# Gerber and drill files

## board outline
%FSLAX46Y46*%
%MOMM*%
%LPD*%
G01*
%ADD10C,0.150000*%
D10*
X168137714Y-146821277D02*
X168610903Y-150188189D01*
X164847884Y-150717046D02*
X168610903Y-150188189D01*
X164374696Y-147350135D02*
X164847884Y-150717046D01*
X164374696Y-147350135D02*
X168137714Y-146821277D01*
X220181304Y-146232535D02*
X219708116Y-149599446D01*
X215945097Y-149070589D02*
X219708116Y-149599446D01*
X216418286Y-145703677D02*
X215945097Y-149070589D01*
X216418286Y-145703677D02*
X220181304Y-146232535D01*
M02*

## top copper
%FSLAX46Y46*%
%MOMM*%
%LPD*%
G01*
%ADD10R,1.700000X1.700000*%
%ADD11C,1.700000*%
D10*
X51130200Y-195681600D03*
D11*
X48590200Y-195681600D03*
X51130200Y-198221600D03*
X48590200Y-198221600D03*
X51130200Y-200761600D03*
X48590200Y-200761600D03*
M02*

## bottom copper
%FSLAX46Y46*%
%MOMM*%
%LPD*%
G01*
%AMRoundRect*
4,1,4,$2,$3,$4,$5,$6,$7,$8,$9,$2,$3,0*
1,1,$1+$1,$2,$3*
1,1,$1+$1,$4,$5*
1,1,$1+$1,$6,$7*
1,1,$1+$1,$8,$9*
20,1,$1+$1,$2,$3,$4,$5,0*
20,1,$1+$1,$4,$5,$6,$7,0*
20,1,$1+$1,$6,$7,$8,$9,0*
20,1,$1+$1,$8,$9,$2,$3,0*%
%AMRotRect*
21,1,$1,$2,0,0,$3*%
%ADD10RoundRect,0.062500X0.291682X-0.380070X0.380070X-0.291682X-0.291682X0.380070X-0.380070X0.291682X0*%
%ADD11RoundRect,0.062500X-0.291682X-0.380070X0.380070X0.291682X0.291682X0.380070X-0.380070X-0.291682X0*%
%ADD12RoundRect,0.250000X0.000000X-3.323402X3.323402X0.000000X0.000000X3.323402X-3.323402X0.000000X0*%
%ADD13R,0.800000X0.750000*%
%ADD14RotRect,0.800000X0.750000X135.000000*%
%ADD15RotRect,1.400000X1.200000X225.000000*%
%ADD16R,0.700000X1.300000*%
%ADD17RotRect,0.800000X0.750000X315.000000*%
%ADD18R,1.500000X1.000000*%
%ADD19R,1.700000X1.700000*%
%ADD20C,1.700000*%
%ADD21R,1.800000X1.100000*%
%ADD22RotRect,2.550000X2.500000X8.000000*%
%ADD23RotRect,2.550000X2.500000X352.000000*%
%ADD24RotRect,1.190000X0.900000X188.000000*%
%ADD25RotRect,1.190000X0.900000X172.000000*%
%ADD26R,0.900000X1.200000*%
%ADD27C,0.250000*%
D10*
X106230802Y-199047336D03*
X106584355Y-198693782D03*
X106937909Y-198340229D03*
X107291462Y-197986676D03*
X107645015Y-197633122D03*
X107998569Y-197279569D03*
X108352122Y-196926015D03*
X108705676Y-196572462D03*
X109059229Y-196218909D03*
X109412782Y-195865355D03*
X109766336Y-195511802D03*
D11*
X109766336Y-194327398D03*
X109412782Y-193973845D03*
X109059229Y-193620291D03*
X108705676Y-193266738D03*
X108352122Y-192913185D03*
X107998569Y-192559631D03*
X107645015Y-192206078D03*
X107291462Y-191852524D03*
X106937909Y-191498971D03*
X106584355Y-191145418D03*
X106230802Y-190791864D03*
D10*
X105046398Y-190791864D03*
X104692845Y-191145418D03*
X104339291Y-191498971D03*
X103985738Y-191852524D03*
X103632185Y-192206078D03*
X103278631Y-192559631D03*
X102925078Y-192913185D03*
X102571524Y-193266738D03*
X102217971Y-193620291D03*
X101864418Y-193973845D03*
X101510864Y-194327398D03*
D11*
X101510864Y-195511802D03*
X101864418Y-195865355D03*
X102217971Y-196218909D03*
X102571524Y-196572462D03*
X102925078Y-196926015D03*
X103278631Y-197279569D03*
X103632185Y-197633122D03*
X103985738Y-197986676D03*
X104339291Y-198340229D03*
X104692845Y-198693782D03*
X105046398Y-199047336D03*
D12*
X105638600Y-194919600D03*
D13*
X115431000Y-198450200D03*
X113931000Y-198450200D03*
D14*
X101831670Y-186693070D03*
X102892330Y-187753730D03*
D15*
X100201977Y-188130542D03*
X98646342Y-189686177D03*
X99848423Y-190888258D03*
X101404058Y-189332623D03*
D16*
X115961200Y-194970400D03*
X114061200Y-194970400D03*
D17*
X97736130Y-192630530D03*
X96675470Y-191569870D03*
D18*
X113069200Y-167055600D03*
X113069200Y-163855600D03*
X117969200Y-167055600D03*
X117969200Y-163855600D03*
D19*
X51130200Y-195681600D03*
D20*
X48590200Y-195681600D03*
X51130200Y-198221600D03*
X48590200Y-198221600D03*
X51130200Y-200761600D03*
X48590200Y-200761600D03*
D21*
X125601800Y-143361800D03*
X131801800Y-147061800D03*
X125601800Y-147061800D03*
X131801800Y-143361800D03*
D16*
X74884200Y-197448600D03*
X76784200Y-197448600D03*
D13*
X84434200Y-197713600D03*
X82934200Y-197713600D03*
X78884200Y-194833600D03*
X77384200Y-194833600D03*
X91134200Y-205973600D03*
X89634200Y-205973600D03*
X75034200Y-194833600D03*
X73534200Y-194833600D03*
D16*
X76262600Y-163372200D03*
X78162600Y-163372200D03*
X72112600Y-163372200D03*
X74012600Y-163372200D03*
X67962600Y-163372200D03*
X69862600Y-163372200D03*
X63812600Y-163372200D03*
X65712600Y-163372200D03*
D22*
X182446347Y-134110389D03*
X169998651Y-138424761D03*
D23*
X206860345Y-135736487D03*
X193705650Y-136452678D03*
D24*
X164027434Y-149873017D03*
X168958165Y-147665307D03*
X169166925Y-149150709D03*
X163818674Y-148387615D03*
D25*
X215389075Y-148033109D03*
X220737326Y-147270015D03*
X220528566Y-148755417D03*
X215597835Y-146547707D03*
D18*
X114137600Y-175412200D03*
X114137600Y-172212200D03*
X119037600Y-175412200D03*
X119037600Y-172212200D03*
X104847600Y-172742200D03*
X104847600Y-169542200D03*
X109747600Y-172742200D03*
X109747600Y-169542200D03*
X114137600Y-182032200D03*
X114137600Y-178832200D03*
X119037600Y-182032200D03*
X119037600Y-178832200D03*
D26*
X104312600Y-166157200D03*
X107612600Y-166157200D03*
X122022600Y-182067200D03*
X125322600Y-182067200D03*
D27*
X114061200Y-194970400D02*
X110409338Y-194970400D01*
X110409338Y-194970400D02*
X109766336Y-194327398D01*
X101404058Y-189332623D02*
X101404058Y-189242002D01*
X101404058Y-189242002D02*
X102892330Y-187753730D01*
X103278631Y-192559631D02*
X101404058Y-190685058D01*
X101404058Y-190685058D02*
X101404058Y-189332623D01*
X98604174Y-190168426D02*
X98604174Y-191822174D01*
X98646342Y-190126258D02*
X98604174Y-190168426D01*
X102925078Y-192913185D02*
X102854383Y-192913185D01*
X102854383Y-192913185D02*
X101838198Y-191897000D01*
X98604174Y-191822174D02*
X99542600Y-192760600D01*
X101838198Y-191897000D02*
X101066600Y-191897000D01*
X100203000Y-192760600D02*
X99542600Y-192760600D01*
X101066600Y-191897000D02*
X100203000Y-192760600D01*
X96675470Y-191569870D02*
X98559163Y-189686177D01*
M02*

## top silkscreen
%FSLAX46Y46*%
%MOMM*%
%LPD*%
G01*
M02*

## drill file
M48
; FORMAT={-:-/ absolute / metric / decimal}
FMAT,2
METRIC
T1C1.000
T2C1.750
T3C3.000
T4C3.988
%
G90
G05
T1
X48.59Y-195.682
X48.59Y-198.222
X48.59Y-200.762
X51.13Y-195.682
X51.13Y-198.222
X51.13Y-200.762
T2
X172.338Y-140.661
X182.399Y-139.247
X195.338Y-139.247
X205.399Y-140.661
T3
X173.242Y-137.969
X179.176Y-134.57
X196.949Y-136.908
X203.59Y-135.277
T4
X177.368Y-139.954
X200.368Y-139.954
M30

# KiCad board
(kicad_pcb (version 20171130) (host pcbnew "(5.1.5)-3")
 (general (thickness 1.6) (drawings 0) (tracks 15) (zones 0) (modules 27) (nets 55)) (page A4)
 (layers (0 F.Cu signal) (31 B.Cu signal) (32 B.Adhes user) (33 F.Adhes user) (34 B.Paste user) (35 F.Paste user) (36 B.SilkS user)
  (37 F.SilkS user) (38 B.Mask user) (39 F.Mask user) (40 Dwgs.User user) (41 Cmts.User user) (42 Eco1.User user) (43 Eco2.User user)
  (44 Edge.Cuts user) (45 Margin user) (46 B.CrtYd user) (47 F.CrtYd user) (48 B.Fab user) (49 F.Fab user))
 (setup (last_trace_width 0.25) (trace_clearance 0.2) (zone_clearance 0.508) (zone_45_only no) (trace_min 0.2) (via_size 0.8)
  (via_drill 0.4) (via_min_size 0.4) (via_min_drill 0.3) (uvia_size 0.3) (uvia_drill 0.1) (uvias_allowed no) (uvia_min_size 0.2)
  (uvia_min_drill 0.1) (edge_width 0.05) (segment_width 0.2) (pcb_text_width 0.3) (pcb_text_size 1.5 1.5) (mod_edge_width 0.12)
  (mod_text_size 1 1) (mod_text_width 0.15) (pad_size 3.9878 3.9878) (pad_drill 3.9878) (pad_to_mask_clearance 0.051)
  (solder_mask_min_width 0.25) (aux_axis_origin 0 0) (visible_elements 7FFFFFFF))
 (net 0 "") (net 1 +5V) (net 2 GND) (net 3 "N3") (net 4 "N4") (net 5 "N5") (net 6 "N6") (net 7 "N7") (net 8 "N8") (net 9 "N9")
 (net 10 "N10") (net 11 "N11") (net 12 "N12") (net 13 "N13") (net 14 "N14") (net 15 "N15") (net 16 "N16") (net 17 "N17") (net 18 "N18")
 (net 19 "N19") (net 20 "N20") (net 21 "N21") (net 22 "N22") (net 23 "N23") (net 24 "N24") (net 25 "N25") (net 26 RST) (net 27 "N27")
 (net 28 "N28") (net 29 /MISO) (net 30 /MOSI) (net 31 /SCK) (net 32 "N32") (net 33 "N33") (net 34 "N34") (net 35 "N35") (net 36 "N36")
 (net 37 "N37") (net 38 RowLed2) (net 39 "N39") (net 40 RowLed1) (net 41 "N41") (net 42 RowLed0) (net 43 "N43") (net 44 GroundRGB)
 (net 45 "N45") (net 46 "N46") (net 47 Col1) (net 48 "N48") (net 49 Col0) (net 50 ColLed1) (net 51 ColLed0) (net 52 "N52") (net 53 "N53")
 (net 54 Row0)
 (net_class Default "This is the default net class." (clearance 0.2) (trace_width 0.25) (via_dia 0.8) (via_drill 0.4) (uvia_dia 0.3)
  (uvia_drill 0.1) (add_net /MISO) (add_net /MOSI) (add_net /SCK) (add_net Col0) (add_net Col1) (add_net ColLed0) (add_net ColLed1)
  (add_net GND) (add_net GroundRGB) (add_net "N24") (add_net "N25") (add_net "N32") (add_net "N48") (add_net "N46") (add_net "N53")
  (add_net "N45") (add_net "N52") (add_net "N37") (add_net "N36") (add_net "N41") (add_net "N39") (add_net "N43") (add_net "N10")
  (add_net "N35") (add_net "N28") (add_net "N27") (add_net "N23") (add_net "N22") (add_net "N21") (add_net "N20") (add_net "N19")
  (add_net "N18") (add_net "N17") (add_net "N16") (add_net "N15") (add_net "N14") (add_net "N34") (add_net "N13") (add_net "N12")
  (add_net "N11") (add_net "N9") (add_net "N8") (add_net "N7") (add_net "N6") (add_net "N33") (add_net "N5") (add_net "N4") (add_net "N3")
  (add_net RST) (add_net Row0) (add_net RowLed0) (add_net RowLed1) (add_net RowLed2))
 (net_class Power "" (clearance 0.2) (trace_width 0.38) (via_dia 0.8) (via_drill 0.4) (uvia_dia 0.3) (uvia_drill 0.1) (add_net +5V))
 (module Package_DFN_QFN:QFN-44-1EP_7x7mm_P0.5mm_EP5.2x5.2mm (layer B.Cu) (at 105.6386 194.9196 45)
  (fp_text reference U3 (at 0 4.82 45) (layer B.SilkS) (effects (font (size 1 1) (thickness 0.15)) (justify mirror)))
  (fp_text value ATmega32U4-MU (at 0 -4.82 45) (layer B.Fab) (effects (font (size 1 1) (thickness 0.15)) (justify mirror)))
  (pad 44 smd roundrect (at -2.5 3.3375 45) (size 0.25 1.075) (layers B.Cu B.Paste B.Mask) (roundrect_rratio 0.25) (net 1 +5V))
  (pad 43 smd roundrect (at -2 3.3375 45) (size 0.25 1.075) (layers B.Cu B.Paste B.Mask) (roundrect_rratio 0.25) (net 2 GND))
  (pad 42 smd roundrect (at -1.5 3.3375 45) (size 0.25 1.075) (layers B.Cu B.Paste B.Mask) (roundrect_rratio 0.25) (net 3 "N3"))
  (pad 41 smd roundrect (at -1 3.3375 45) (size 0.25 1.075) (layers B.Cu B.Paste B.Mask) (roundrect_rratio 0.25) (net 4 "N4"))
  (pad 40 smd roundrect (at -0.5 3.3375 45) (size 0.25 1.075) (layers B.Cu B.Paste B.Mask) (roundrect_rratio 0.25) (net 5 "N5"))
  (pad 39 smd roundrect (at 0 3.3375 45) (size 0.25 1.075) (layers B.Cu B.Paste B.Mask) (roundrect_rratio 0.25) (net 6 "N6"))
  (pad 38 smd roundrect (at 0.5 3.3375 45) (size 0.25 1.075) (layers B.Cu B.Paste B.Mask) (roundrect_rratio 0.25) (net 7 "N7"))
  (pad 37 smd roundrect (at 1 3.3375 45) (size 0.25 1.075) (layers B.Cu B.Paste B.Mask) (roundrect_rratio 0.25) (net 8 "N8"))
  (pad 36 smd roundrect (at 1.5 3.3375 45) (size 0.25 1.075) (layers B.Cu B.Paste B.Mask) (roundrect_rratio 0.25) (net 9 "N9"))
  (pad 35 smd roundrect (at 2 3.3375 45) (size 0.25 1.075) (layers B.Cu B.Paste B.Mask) (roundrect_rratio 0.25) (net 2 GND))
  (pad 34 smd roundrect (at 2.5 3.3375 45) (size 0.25 1.075) (layers B.Cu B.Paste B.Mask) (roundrect_rratio 0.25) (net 1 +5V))
  (pad 33 smd roundrect (at 3.3375 2.5 45) (size 1.075 0.25) (layers B.Cu B.Paste B.Mask) (roundrect_rratio 0.25) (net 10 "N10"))
  (pad 32 smd roundrect (at 3.3375 2 45) (size 1.075 0.25) (layers B.Cu B.Paste B.Mask) (roundrect_rratio 0.25) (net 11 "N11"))
  (pad 31 smd roundrect (at 3.3375 1.5 45) (size 1.075 0.25) (layers B.Cu B.Paste B.Mask) (roundrect_rratio 0.25) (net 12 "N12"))
  (pad 30 smd roundrect (at 3.3375 1 45) (size 1.075 0.25) (layers B.Cu B.Paste B.Mask) (roundrect_rratio 0.25) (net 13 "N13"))
  (pad 29 smd roundrect (at 3.3375 0.5 45) (size 1.075 0.25) (layers B.Cu B.Paste B.Mask) (roundrect_rratio 0.25) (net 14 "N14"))
  (pad 28 smd roundrect (at 3.3375 0 45) (size 1.075 0.25) (layers B.Cu B.Paste B.Mask) (roundrect_rratio 0.25) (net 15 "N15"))
  (pad 27 smd roundrect (at 3.3375 -0.5 45) (size 1.075 0.25) (layers B.Cu B.Paste B.Mask) (roundrect_rratio 0.25) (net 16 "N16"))
  (pad 26 smd roundrect (at 3.3375 -1 45) (size 1.075 0.25) (layers B.Cu B.Paste B.Mask) (roundrect_rratio 0.25) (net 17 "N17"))
  (pad 25 smd roundrect (at 3.3375 -1.5 45) (size 1.075 0.25) (layers B.Cu B.Paste B.Mask) (roundrect_rratio 0.25) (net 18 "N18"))
  (pad 24 smd roundrect (at 3.3375 -2 45) (size 1.075 0.25) (layers B.Cu B.Paste B.Mask) (roundrect_rratio 0.25) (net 1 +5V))
  (pad 23 smd roundrect (at 3.3375 -2.5 45) (size 1.075 0.25) (layers B.Cu B.Paste B.Mask) (roundrect_rratio 0.25) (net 2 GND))
  (pad 22 smd roundrect (at 2.5 -3.3375 45) (size 0.25 1.075) (layers B.Cu B.Paste B.Mask) (roundrect_rratio 0.25) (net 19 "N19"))
  (pad 21 smd roundrect (at 2 -3.3375 45) (size 0.25 1.075) (layers B.Cu B.Paste B.Mask) (roundrect_rratio 0.25) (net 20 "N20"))
  (pad 20 smd roundrect (at 1.5 -3.3375 45) (size 0.25 1.075) (layers B.Cu B.Paste B.Mask) (roundrect_rratio 0.25) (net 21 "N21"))
  (pad 19 smd roundrect (at 1 -3.3375 45) (size 0.25 1.075) (layers B.Cu B.Paste B.Mask) (roundrect_rratio 0.25) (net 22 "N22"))
  (pad 18 smd roundrect (at 0.5 -3.3375 45) (size 0.25 1.075) (layers B.Cu B.Paste B.Mask) (roundrect_rratio 0.25) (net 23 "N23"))
  (pad 17 smd roundrect (at 0 -3.3375 45) (size 0.25 1.075) (layers B.Cu B.Paste B.Mask) (roundrect_rratio 0.25) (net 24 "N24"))
  (pad 16 smd roundrect (at -0.5 -3.3375 45) (size 0.25 1.075) (layers B.Cu B.Paste B.Mask) (roundrect_rratio 0.25) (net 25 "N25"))
  (pad 15 smd roundrect (at -1 -3.3375 45) (size 0.25 1.075) (layers B.Cu B.Paste B.Mask) (roundrect_rratio 0.25) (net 2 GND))
  (pad 14 smd roundrect (at -1.5 -3.3375 45) (size 0.25 1.075) (layers B.Cu B.Paste B.Mask) (roundrect_rratio 0.25) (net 1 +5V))
  (pad 13 smd roundrect (at -2 -3.3375 45) (size 0.25 1.075) (layers B.Cu B.Paste B.Mask) (roundrect_rratio 0.25) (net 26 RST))
  (pad 12 smd roundrect (at -2.5 -3.3375 45) (size 0.25 1.075) (layers B.Cu B.Paste B.Mask) (roundrect_rratio 0.25) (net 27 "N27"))
  (pad 11 smd roundrect (at -3.3375 -2.5 45) (size 1.075 0.25) (layers B.Cu B.Paste B.Mask) (roundrect_rratio 0.25) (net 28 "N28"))
  (pad 10 smd roundrect (at -3.3375 -2 45) (size 1.075 0.25) (layers B.Cu B.Paste B.Mask) (roundrect_rratio 0.25) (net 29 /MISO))
  (pad 9 smd roundrect (at -3.3375 -1.5 45) (size 1.075 0.25) (layers B.Cu B.Paste B.Mask) (roundrect_rratio 0.25) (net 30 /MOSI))
  (pad 8 smd roundrect (at -3.3375 -1 45) (size 1.075 0.25) (layers B.Cu B.Paste B.Mask) (roundrect_rratio 0.25) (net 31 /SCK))
  (pad 7 smd roundrect (at -3.3375 -0.5 45) (size 1.075 0.25) (layers B.Cu B.Paste B.Mask) (roundrect_rratio 0.25) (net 1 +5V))
  (pad 6 smd roundrect (at -3.3375 0 45) (size 1.075 0.25) (layers B.Cu B.Paste B.Mask) (roundrect_rratio 0.25) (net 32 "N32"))
  (pad 5 smd roundrect (at -3.3375 0.5 45) (size 1.075 0.25) (layers B.Cu B.Paste B.Mask) (roundrect_rratio 0.25) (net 2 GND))
  (pad 4 smd roundrect (at -3.3375 1 45) (size 1.075 0.25) (layers B.Cu B.Paste B.Mask) (roundrect_rratio 0.25) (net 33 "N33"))
  (pad 3 smd roundrect (at -3.3375 1.5 45) (size 1.075 0.25) (layers B.Cu B.Paste B.Mask) (roundrect_rratio 0.25) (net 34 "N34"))
  (pad 2 smd roundrect (at -3.3375 2 45) (size 1.075 0.25) (layers B.Cu B.Paste B.Mask) (roundrect_rratio 0.25) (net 1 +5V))
  (pad 1 smd roundrect (at -3.3375 2.5 45) (size 1.075 0.25) (layers B.Cu B.Paste B.Mask) (roundrect_rratio 0.25) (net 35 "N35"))
  (pad "" smd roundrect (at 1.95 -1.95 45) (size 1.05 1.05) (layers B.Paste) (roundrect_rratio 0.238095))
  (pad "" smd roundrect (at 1.95 -0.65 45) (size 1.05 1.05) (layers B.Paste) (roundrect_rratio 0.238095))
  (pad "" smd roundrect (at 1.95 0.65 45) (size 1.05 1.05) (layers B.Paste) (roundrect_rratio 0.238095))
  (pad "" smd roundrect (at 1.95 1.95 45) (size 1.05 1.05) (layers B.Paste) (roundrect_rratio 0.238095))
  (pad "" smd roundrect (at 0.65 -1.95 45) (size 1.05 1.05) (layers B.Paste) (roundrect_rratio 0.238095))
  (pad "" smd roundrect (at 0.65 -0.65 45) (size 1.05 1.05) (layers B.Paste) (roundrect_rratio 0.238095))
  (pad "" smd roundrect (at 0.65 0.65 45) (size 1.05 1.05) (layers B.Paste) (roundrect_rratio 0.238095))
  (pad "" smd roundrect (at 0.65 1.95 45) (size 1.05 1.05) (layers B.Paste) (roundrect_rratio 0.238095))
  (pad "" smd roundrect (at -0.65 -1.95 45) (size 1.05 1.05) (layers B.Paste) (roundrect_rratio 0.238095))
  (pad "" smd roundrect (at -0.65 -0.65 45) (size 1.05 1.05) (layers B.Paste) (roundrect_rratio 0.238095))
  (pad "" smd roundrect (at -0.65 0.65 45) (size 1.05 1.05) (layers B.Paste) (roundrect_rratio 0.238095))
  (pad "" smd roundrect (at -0.65 1.95 45) (size 1.05 1.05) (layers B.Paste) (roundrect_rratio 0.238095))
  (pad "" smd roundrect (at -1.95 -1.95 45) (size 1.05 1.05) (layers B.Paste) (roundrect_rratio 0.238095))
  (pad "" smd roundrect (at -1.95 -0.65 45) (size 1.05 1.05) (layers B.Paste) (roundrect_rratio 0.238095))
  (pad "" smd roundrect (at -1.95 0.65 45) (size 1.05 1.05) (layers B.Paste) (roundrect_rratio 0.238095))
  (pad "" smd roundrect (at -1.95 1.95 45) (size 1.05 1.05) (layers B.Paste) (roundrect_rratio 0.238095))
  (pad 45 smd roundrect (at 0 0 45) (size 5.2 5.2) (layers B.Cu B.Mask) (roundrect_rratio 0.048077) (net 2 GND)))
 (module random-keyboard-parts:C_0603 (layer B.Cu) (at 114.681 198.4502)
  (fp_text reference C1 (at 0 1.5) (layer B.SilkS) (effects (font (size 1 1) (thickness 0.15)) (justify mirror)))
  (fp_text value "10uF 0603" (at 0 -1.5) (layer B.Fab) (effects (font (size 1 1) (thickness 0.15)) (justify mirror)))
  (pad 2 smd rect (at 0.75 0) (size 0.8 0.75) (layers B.Cu B.Paste B.Mask) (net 2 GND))
  (pad 1 smd rect (at -0.75 0) (size 0.8 0.75) (layers B.Cu B.Paste B.Mask) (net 1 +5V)))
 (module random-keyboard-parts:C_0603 (layer B.Cu) (at 102.362 187.2234 135)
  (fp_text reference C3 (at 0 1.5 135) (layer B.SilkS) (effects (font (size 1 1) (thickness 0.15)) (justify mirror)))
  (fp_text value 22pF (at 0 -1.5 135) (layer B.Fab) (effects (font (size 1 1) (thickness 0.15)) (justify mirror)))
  (pad 2 smd rect (at 0.75 0 135) (size 0.8 0.75) (layers B.Cu B.Paste B.Mask) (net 2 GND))
  (pad 1 smd rect (at -0.75 0 135) (size 0.8 0.75) (layers B.Cu B.Paste B.Mask) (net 24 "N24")))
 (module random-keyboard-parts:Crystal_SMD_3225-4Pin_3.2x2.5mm (layer B.Cu) (at 100.0252 189.5094 225)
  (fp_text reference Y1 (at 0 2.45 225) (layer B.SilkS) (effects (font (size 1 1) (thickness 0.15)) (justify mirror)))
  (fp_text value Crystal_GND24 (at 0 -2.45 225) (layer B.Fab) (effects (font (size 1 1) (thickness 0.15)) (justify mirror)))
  (pad 4 smd rect (at -1.1 0.85 225) (size 1.4 1.2) (layers B.Cu B.Paste B.Mask) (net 2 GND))
  (pad 3 smd rect (at 1.1 0.85 225) (size 1.4 1.2) (layers B.Cu B.Paste B.Mask) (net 25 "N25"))
  (pad 2 smd rect (at 1.1 -0.85 225) (size 1.4 1.2) (layers B.Cu B.Paste B.Mask) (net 2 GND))
  (pad 1 smd rect (at -1.1 -0.85 225) (size 1.4 1.2) (layers B.Cu B.Paste B.Mask) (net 24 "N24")))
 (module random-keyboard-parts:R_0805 (layer B.Cu) (at 115.0112 194.9704 180)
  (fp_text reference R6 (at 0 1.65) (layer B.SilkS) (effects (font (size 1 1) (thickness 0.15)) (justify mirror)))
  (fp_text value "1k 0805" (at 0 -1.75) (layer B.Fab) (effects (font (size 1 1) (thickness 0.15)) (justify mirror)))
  (pad 1 smd rect (at -0.95 0 180) (size 0.7 1.3) (layers B.Cu B.Paste B.Mask) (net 2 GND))
  (pad 2 smd rect (at 0.95 0 180) (size 0.7 1.3) (layers B.Cu B.Paste B.Mask) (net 10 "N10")))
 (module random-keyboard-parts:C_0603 (layer B.Cu) (at 97.2058 192.1002 315)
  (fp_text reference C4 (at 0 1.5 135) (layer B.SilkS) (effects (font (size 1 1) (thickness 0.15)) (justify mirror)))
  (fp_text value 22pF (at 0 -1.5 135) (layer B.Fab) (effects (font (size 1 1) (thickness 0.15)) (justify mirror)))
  (pad 2 smd rect (at 0.75 0 315) (size 0.8 0.75) (layers B.Cu B.Paste B.Mask) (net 2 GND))
  (pad 1 smd rect (at -0.75 0 315) (size 0.8 0.75) (layers B.Cu B.Paste B.Mask) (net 25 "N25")))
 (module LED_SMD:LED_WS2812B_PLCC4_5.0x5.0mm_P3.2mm (layer B.Cu) (at 115.5192 165.4556)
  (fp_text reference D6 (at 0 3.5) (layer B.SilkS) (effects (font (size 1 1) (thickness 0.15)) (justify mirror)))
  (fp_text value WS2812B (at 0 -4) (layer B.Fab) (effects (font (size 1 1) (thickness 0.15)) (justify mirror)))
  (pad 1 smd rect (at -2.45 1.6) (size 1.5 1) (layers B.Cu B.Paste B.Mask) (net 2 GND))
  (pad 2 smd rect (at -2.45 -1.6) (size 1.5 1) (layers B.Cu B.Paste B.Mask) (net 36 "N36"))
  (pad 4 smd rect (at 2.45 1.6) (size 1.5 1) (layers B.Cu B.Paste B.Mask) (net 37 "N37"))
  (pad 3 smd rect (at 2.45 -1.6) (size 1.5 1) (layers B.Cu B.Paste B.Mask) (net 1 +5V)))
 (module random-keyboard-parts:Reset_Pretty (layer B.Cu) (at 49.8602 198.2216)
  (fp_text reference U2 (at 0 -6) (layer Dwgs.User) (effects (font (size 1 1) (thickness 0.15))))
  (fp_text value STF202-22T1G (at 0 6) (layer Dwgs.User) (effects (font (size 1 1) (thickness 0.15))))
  (pad 6 thru_hole rect (at 1.27 -2.54) (size 1.7 1.7) (drill 1) (layers *.Cu *.Mask) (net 2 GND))
  (pad 5 thru_hole circle (at -1.27 -2.54) (size 1.7 1.7) (drill 1) (layers *.Cu *.Mask) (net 26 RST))
  (pad 4 thru_hole circle (at 1.27 0) (size 1.7 1.7) (drill 1) (layers *.Cu *.Mask) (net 30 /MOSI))
  (pad 3 thru_hole circle (at -1.27 0) (size 1.7 1.7) (drill 1) (layers *.Cu *.Mask) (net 31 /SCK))
  (pad 2 thru_hole circle (at 1.27 2.54) (size 1.7 1.7) (drill 1) (layers *.Cu *.Mask) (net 1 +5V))
  (pad 1 thru_hole circle (at -1.27 2.54) (size 1.7 1.7) (drill 1) (layers *.Cu *.Mask) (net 29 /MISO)))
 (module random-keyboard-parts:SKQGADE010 (layer B.Cu) (at 128.7018 145.2118)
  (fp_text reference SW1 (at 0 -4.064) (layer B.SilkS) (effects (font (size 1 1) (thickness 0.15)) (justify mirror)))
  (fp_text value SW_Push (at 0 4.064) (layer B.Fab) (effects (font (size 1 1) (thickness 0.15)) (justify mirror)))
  (pad 4 smd rect (at -3.1 -1.85) (size 1.8 1.1) (layers B.Cu B.Paste B.Mask))
  (pad 3 smd rect (at 3.1 1.85) (size 1.8 1.1) (layers B.Cu B.Paste B.Mask))
  (pad 2 smd rect (at -3.1 1.85) (size 1.8 1.1) (layers B.Cu B.Paste B.Mask) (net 26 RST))
  (pad 1 smd rect (at 3.1 -1.85) (size 1.8 1.1) (layers B.Cu B.Paste B.Mask) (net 2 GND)))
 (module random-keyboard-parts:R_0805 (layer B.Cu) (at 75.8342 197.4486)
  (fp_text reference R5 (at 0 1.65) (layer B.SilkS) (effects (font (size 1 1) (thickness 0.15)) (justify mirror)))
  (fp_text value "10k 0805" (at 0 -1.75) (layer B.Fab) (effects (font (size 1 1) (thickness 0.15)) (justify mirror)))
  (pad 1 smd rect (at -0.95 0) (size 0.7 1.3) (layers B.Cu B.Paste B.Mask) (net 1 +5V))
  (pad 2 smd rect (at 0.95 0) (size 0.7 1.3) (layers B.Cu B.Paste B.Mask) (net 26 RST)))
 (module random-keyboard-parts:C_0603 (layer B.Cu) (at 83.6842 197.7136)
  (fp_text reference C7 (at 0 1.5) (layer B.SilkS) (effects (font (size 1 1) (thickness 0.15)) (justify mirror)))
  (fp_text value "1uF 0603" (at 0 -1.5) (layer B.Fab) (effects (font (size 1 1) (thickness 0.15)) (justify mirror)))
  (pad 2 smd rect (at 0.75 0) (size 0.8 0.75) (layers B.Cu B.Paste B.Mask) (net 2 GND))
  (pad 1 smd rect (at -0.75 0) (size 0.8 0.75) (layers B.Cu B.Paste B.Mask) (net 32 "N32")))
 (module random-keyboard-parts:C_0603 (layer B.Cu) (at 78.1342 194.8336)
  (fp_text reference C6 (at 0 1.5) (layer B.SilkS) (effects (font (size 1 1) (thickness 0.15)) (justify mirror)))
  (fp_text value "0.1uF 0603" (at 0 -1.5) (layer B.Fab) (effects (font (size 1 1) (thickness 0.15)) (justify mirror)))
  (pad 2 smd rect (at 0.75 0) (size 0.8 0.75) (layers B.Cu B.Paste B.Mask) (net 2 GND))
  (pad 1 smd rect (at -0.75 0) (size 0.8 0.75) (layers B.Cu B.Paste B.Mask) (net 1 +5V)))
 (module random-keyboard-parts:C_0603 (layer B.Cu) (at 90.3842 205.9736)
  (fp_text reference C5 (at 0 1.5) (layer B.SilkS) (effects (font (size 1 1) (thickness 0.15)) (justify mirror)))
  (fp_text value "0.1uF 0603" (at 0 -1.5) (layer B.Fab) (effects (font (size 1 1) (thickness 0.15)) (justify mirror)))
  (pad 2 smd rect (at 0.75 0) (size 0.8 0.75) (layers B.Cu B.Paste B.Mask) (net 2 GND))
  (pad 1 smd rect (at -0.75 0) (size 0.8 0.75) (layers B.Cu B.Paste B.Mask) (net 1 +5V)))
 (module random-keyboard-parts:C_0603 (layer B.Cu) (at 74.2842 194.8336)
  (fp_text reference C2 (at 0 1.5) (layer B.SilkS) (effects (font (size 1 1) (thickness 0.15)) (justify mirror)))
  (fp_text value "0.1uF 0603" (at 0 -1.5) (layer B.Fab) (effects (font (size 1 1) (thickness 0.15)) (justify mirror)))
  (pad 2 smd rect (at 0.75 0) (size 0.8 0.75) (layers B.Cu B.Paste B.Mask) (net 2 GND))
  (pad 1 smd rect (at -0.75 0) (size 0.8 0.75) (layers B.Cu B.Paste B.Mask) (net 1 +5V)))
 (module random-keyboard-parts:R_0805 (layer B.Cu) (at 77.2126 163.3722)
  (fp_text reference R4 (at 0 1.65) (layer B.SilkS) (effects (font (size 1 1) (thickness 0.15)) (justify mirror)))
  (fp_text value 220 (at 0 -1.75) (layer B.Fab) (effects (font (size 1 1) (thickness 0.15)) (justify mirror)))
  (pad 1 smd rect (at -0.95 0) (size 0.7 1.3) (layers B.Cu B.Paste B.Mask) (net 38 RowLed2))
  (pad 2 smd rect (at 0.95 0) (size 0.7 1.3) (layers B.Cu B.Paste B.Mask) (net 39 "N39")))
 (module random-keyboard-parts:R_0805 (layer B.Cu) (at 73.0626 163.3722)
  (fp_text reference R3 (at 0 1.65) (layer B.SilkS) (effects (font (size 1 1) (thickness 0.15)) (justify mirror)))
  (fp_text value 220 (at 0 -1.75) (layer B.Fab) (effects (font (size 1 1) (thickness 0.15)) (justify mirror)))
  (pad 1 smd rect (at -0.95 0) (size 0.7 1.3) (layers B.Cu B.Paste B.Mask) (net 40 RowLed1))
  (pad 2 smd rect (at 0.95 0) (size 0.7 1.3) (layers B.Cu B.Paste B.Mask) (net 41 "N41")))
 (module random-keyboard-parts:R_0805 (layer B.Cu) (at 68.9126 163.3722)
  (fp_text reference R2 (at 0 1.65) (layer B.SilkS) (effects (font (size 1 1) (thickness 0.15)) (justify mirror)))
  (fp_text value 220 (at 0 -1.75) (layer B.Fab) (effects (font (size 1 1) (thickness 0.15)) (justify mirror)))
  (pad 1 smd rect (at -0.95 0) (size 0.7 1.3) (layers B.Cu B.Paste B.Mask) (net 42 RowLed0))
  (pad 2 smd rect (at 0.95 0) (size 0.7 1.3) (layers B.Cu B.Paste B.Mask) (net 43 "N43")))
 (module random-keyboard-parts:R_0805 (layer B.Cu) (at 64.7626 163.3722)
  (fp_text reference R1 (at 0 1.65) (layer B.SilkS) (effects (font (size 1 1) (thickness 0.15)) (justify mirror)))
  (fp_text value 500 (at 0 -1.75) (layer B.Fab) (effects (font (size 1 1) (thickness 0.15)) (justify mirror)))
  (pad 1 smd rect (at -0.95 0) (size 0.7 1.3) (layers B.Cu B.Paste B.Mask) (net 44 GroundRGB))
  (pad 2 smd rect (at 0.95 0) (size 0.7 1.3) (layers B.Cu B.Paste B.Mask) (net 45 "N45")))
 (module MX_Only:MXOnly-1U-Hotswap (layer F.Cu) (at 177.3682 139.954 8)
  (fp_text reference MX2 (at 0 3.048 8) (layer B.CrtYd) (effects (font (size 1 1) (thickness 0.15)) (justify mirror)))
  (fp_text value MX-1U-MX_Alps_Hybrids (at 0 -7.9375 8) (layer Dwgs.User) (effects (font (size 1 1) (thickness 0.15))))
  (pad 2 smd rect (at 5.842 -5.08 8) (size 2.55 2.5) (layers B.Cu B.Paste B.Mask) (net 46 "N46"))
  (pad 1 smd rect (at -7.085 -2.54 8) (size 2.55 2.5) (layers B.Cu B.Paste B.Mask) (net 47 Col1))
  (pad "" np_thru_hole circle (at 5.08 0 56.0996) (size 1.75 1.75) (drill 1.75) (layers *.Cu *.Mask))
  (pad "" np_thru_hole circle (at -5.08 0 56.0996) (size 1.75 1.75) (drill 1.75) (layers *.Cu *.Mask))
  (pad "" np_thru_hole circle (at -3.81 -2.54 8) (size 3 3) (drill 3) (layers *.Cu *.Mask))
  (pad "" np_thru_hole circle (at 0 0 8) (size 3.9878 3.9878) (drill 3.9878) (layers *.Cu *.Mask))
  (pad "" np_thru_hole circle (at 2.54 -5.08 8) (size 3 3) (drill 3) (layers *.Cu *.Mask)))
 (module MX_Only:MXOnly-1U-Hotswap (layer F.Cu) (at 200.3682 139.954 352)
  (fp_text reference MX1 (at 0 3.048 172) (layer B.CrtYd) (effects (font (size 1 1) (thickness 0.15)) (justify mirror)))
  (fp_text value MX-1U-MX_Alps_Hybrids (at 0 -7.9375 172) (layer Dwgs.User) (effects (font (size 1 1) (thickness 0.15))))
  (pad 2 smd rect (at 5.842 -5.08 352) (size 2.55 2.5) (layers B.Cu B.Paste B.Mask) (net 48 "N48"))
  (pad 1 smd rect (at -7.085 -2.54 352) (size 2.55 2.5) (layers B.Cu B.Paste B.Mask) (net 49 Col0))
  (pad "" np_thru_hole circle (at 5.08 0 40.0996) (size 1.75 1.75) (drill 1.75) (layers *.Cu *.Mask))
  (pad "" np_thru_hole circle (at -5.08 0 40.0996) (size 1.75 1.75) (drill 1.75) (layers *.Cu *.Mask))
  (pad "" np_thru_hole circle (at -3.81 -2.54 352) (size 3 3) (drill 3) (layers *.Cu *.Mask))
  (pad "" np_thru_hole circle (at 0 0 352) (size 3.9878 3.9878) (drill 3.9878) (layers *.Cu *.Mask))
  (pad "" np_thru_hole circle (at 2.54 -5.08 352) (size 3 3) (drill 3) (layers *.Cu *.Mask)))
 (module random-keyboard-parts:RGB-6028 (layer B.Cu) (at 165.7858 143.7386 188)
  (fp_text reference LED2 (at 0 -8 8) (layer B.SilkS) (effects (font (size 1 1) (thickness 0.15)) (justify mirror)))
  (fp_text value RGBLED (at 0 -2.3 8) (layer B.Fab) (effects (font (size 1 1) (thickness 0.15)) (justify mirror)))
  (fp_line (start -1.9 -3.38) (end -1.9 -6.78) (layer Edge.Cuts) (width 0.15))
  (fp_line (start 1.9 -6.78) (end -1.9 -6.78) (layer Edge.Cuts) (width 0.15))
  (fp_line (start 1.9 -3.38) (end 1.9 -6.78) (layer Edge.Cuts) (width 0.15))
  (fp_line (start 1.9 -3.38) (end -1.9 -3.38) (layer Edge.Cuts) (width 0.15))
  (pad 2 smd rect (at 2.595 -5.83 188) (size 1.19 0.9) (layers B.Cu B.Paste B.Mask) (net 41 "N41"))
  (pad 1 smd rect (at -2.595 -4.33 188) (size 1.19 0.9) (layers B.Cu B.Paste B.Mask) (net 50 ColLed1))
  (pad 4 smd rect (at -2.595 -5.83 188) (size 1.19 0.9) (layers B.Cu B.Paste B.Mask) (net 43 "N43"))
  (pad 3 smd rect (at 2.595 -4.33 188) (size 1.19 0.9) (layers B.Cu B.Paste B.Mask) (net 39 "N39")))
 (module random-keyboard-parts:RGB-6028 (layer B.Cu) (at 218.7702 142.621 172)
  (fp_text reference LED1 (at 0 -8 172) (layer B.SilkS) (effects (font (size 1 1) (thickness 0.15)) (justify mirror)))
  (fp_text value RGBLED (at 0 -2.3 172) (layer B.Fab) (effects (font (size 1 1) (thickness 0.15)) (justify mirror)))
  (fp_line (start -1.9 -3.38) (end -1.9 -6.78) (layer Edge.Cuts) (width 0.15))
  (fp_line (start 1.9 -6.78) (end -1.9 -6.78) (layer Edge.Cuts) (width 0.15))
  (fp_line (start 1.9 -3.38) (end 1.9 -6.78) (layer Edge.Cuts) (width 0.15))
  (fp_line (start 1.9 -3.38) (end -1.9 -3.38) (layer Edge.Cuts) (width 0.15))
  (pad 2 smd rect (at 2.595 -5.83 172) (size 1.19 0.9) (layers B.Cu B.Paste B.Mask) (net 41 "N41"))
  (pad 1 smd rect (at -2.595 -4.33 172) (size 1.19 0.9) (layers B.Cu B.Paste B.Mask) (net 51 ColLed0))
  (pad 4 smd rect (at -2.595 -5.83 172) (size 1.19 0.9) (layers B.Cu B.Paste B.Mask) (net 43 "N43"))
  (pad 3 smd rect (at 2.595 -4.33 172) (size 1.19 0.9) (layers B.Cu B.Paste B.Mask) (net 39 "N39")))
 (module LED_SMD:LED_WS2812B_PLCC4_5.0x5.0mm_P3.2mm (layer B.Cu) (at 116.5876 173.8122)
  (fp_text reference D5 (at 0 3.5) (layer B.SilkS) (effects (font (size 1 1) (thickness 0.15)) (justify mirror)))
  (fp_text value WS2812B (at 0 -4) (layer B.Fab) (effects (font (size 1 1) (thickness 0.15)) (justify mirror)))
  (pad 1 smd rect (at -2.45 1.6) (size 1.5 1) (layers B.Cu B.Paste B.Mask) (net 2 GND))
  (pad 2 smd rect (at -2.45 -1.6) (size 1.5 1) (layers B.Cu B.Paste B.Mask) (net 37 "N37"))
  (pad 4 smd rect (at 2.45 1.6) (size 1.5 1) (layers B.Cu B.Paste B.Mask) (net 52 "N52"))
  (pad 3 smd rect (at 2.45 -1.6) (size 1.5 1) (layers B.Cu B.Paste B.Mask) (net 1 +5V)))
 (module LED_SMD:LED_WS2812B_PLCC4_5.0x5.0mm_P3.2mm (layer B.Cu) (at 107.2976 171.1422)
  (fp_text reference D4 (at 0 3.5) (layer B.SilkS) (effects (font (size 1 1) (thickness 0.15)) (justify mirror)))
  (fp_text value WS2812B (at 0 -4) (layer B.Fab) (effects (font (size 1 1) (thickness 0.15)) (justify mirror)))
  (pad 1 smd rect (at -2.45 1.6) (size 1.5 1) (layers B.Cu B.Paste B.Mask) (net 2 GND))
  (pad 2 smd rect (at -2.45 -1.6) (size 1.5 1) (layers B.Cu B.Paste B.Mask) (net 52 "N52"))
  (pad 4 smd rect (at 2.45 1.6) (size 1.5 1) (layers B.Cu B.Paste B.Mask) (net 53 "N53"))
  (pad 3 smd rect (at 2.45 -1.6) (size 1.5 1) (layers B.Cu B.Paste B.Mask) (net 1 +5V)))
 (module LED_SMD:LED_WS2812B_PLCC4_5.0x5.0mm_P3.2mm (layer B.Cu) (at 116.5876 180.4322)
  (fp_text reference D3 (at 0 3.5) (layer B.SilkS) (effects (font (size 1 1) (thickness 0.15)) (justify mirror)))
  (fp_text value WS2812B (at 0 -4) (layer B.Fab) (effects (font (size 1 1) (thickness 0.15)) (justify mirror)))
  (pad 1 smd rect (at -2.45 1.6) (size 1.5 1) (layers B.Cu B.Paste B.Mask) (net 2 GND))
  (pad 2 smd rect (at -2.45 -1.6) (size 1.5 1) (layers B.Cu B.Paste B.Mask) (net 53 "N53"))
  (pad 4 smd rect (at 2.45 1.6) (size 1.5 1) (layers B.Cu B.Paste B.Mask) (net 45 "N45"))
  (pad 3 smd rect (at 2.45 -1.6) (size 1.5 1) (layers B.Cu B.Paste B.Mask) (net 1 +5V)))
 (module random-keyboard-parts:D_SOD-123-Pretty (layer B.Cu) (at 105.9626 166.1572)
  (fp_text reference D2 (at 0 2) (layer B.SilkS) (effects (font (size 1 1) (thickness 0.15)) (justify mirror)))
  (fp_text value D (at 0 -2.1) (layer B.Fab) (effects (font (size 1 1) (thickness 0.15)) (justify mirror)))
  (pad 1 smd rect (at -1.65 0) (size 0.9 1.2) (layers B.Cu B.Paste B.Mask) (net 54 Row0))
  (pad 2 smd rect (at 1.65 0) (size 0.9 1.2) (layers B.Cu B.Paste B.Mask) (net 46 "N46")))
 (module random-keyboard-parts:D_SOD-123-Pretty (layer B.Cu) (at 123.6726 182.0672)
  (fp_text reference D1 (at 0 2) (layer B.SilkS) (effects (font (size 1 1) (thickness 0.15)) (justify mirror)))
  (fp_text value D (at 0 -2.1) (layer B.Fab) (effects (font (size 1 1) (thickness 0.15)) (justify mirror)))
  (pad 1 smd rect (at -1.65 0) (size 0.9 1.2) (layers B.Cu B.Paste B.Mask) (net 54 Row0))
  (pad 2 smd rect (at 1.65 0) (size 0.9 1.2) (layers B.Cu B.Paste B.Mask) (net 48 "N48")))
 (segment (start 114.0612 194.9704) (end 110.409338 194.9704) (width 0.25) (layer B.Cu) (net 10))
 (segment (start 110.409338 194.9704) (end 109.766336 194.327398) (width 0.25) (layer B.Cu) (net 10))
 (segment (start 101.404058 189.332623) (end 101.404058 189.242002) (width 0.25) (layer B.Cu) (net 24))
 (segment (start 101.404058 189.242002) (end 102.89233 187.75373) (width 0.25) (layer B.Cu) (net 24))
 (segment (start 103.278631 192.559631) (end 101.404058 190.685058) (width 0.25) (layer B.Cu) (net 24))
 (segment (start 101.404058 190.685058) (end 101.404058 189.332623) (width 0.25) (layer B.Cu) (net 24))
 (segment (start 98.604174 190.168426) (end 98.604174 191.822174) (width 0.25) (layer B.Cu) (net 25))
 (segment (start 98.646342 190.126258) (end 98.604174 190.168426) (width 0.25) (layer B.Cu) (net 25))
 (segment (start 102.925078 192.913185) (end 102.854383 192.913185) (width 0.25) (layer B.Cu) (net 25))
 (segment (start 102.854383 192.913185) (end 101.838198 191.897) (width 0.25) (layer B.Cu) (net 25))
 (segment (start 98.604174 191.822174) (end 99.5426 192.7606) (width 0.25) (layer B.Cu) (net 25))
 (segment (start 101.838198 191.897) (end 101.0666 191.897) (width 0.25) (layer B.Cu) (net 25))
 (segment (start 100.203 192.7606) (end 99.5426 192.7606) (width 0.25) (layer B.Cu) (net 25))
 (segment (start 101.0666 191.897) (end 100.203 192.7606) (width 0.25) (layer B.Cu) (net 25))
 (segment (start 96.67547 191.56987) (end 98.559163 189.686177) (width 0.25) (layer B.Cu) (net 25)))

